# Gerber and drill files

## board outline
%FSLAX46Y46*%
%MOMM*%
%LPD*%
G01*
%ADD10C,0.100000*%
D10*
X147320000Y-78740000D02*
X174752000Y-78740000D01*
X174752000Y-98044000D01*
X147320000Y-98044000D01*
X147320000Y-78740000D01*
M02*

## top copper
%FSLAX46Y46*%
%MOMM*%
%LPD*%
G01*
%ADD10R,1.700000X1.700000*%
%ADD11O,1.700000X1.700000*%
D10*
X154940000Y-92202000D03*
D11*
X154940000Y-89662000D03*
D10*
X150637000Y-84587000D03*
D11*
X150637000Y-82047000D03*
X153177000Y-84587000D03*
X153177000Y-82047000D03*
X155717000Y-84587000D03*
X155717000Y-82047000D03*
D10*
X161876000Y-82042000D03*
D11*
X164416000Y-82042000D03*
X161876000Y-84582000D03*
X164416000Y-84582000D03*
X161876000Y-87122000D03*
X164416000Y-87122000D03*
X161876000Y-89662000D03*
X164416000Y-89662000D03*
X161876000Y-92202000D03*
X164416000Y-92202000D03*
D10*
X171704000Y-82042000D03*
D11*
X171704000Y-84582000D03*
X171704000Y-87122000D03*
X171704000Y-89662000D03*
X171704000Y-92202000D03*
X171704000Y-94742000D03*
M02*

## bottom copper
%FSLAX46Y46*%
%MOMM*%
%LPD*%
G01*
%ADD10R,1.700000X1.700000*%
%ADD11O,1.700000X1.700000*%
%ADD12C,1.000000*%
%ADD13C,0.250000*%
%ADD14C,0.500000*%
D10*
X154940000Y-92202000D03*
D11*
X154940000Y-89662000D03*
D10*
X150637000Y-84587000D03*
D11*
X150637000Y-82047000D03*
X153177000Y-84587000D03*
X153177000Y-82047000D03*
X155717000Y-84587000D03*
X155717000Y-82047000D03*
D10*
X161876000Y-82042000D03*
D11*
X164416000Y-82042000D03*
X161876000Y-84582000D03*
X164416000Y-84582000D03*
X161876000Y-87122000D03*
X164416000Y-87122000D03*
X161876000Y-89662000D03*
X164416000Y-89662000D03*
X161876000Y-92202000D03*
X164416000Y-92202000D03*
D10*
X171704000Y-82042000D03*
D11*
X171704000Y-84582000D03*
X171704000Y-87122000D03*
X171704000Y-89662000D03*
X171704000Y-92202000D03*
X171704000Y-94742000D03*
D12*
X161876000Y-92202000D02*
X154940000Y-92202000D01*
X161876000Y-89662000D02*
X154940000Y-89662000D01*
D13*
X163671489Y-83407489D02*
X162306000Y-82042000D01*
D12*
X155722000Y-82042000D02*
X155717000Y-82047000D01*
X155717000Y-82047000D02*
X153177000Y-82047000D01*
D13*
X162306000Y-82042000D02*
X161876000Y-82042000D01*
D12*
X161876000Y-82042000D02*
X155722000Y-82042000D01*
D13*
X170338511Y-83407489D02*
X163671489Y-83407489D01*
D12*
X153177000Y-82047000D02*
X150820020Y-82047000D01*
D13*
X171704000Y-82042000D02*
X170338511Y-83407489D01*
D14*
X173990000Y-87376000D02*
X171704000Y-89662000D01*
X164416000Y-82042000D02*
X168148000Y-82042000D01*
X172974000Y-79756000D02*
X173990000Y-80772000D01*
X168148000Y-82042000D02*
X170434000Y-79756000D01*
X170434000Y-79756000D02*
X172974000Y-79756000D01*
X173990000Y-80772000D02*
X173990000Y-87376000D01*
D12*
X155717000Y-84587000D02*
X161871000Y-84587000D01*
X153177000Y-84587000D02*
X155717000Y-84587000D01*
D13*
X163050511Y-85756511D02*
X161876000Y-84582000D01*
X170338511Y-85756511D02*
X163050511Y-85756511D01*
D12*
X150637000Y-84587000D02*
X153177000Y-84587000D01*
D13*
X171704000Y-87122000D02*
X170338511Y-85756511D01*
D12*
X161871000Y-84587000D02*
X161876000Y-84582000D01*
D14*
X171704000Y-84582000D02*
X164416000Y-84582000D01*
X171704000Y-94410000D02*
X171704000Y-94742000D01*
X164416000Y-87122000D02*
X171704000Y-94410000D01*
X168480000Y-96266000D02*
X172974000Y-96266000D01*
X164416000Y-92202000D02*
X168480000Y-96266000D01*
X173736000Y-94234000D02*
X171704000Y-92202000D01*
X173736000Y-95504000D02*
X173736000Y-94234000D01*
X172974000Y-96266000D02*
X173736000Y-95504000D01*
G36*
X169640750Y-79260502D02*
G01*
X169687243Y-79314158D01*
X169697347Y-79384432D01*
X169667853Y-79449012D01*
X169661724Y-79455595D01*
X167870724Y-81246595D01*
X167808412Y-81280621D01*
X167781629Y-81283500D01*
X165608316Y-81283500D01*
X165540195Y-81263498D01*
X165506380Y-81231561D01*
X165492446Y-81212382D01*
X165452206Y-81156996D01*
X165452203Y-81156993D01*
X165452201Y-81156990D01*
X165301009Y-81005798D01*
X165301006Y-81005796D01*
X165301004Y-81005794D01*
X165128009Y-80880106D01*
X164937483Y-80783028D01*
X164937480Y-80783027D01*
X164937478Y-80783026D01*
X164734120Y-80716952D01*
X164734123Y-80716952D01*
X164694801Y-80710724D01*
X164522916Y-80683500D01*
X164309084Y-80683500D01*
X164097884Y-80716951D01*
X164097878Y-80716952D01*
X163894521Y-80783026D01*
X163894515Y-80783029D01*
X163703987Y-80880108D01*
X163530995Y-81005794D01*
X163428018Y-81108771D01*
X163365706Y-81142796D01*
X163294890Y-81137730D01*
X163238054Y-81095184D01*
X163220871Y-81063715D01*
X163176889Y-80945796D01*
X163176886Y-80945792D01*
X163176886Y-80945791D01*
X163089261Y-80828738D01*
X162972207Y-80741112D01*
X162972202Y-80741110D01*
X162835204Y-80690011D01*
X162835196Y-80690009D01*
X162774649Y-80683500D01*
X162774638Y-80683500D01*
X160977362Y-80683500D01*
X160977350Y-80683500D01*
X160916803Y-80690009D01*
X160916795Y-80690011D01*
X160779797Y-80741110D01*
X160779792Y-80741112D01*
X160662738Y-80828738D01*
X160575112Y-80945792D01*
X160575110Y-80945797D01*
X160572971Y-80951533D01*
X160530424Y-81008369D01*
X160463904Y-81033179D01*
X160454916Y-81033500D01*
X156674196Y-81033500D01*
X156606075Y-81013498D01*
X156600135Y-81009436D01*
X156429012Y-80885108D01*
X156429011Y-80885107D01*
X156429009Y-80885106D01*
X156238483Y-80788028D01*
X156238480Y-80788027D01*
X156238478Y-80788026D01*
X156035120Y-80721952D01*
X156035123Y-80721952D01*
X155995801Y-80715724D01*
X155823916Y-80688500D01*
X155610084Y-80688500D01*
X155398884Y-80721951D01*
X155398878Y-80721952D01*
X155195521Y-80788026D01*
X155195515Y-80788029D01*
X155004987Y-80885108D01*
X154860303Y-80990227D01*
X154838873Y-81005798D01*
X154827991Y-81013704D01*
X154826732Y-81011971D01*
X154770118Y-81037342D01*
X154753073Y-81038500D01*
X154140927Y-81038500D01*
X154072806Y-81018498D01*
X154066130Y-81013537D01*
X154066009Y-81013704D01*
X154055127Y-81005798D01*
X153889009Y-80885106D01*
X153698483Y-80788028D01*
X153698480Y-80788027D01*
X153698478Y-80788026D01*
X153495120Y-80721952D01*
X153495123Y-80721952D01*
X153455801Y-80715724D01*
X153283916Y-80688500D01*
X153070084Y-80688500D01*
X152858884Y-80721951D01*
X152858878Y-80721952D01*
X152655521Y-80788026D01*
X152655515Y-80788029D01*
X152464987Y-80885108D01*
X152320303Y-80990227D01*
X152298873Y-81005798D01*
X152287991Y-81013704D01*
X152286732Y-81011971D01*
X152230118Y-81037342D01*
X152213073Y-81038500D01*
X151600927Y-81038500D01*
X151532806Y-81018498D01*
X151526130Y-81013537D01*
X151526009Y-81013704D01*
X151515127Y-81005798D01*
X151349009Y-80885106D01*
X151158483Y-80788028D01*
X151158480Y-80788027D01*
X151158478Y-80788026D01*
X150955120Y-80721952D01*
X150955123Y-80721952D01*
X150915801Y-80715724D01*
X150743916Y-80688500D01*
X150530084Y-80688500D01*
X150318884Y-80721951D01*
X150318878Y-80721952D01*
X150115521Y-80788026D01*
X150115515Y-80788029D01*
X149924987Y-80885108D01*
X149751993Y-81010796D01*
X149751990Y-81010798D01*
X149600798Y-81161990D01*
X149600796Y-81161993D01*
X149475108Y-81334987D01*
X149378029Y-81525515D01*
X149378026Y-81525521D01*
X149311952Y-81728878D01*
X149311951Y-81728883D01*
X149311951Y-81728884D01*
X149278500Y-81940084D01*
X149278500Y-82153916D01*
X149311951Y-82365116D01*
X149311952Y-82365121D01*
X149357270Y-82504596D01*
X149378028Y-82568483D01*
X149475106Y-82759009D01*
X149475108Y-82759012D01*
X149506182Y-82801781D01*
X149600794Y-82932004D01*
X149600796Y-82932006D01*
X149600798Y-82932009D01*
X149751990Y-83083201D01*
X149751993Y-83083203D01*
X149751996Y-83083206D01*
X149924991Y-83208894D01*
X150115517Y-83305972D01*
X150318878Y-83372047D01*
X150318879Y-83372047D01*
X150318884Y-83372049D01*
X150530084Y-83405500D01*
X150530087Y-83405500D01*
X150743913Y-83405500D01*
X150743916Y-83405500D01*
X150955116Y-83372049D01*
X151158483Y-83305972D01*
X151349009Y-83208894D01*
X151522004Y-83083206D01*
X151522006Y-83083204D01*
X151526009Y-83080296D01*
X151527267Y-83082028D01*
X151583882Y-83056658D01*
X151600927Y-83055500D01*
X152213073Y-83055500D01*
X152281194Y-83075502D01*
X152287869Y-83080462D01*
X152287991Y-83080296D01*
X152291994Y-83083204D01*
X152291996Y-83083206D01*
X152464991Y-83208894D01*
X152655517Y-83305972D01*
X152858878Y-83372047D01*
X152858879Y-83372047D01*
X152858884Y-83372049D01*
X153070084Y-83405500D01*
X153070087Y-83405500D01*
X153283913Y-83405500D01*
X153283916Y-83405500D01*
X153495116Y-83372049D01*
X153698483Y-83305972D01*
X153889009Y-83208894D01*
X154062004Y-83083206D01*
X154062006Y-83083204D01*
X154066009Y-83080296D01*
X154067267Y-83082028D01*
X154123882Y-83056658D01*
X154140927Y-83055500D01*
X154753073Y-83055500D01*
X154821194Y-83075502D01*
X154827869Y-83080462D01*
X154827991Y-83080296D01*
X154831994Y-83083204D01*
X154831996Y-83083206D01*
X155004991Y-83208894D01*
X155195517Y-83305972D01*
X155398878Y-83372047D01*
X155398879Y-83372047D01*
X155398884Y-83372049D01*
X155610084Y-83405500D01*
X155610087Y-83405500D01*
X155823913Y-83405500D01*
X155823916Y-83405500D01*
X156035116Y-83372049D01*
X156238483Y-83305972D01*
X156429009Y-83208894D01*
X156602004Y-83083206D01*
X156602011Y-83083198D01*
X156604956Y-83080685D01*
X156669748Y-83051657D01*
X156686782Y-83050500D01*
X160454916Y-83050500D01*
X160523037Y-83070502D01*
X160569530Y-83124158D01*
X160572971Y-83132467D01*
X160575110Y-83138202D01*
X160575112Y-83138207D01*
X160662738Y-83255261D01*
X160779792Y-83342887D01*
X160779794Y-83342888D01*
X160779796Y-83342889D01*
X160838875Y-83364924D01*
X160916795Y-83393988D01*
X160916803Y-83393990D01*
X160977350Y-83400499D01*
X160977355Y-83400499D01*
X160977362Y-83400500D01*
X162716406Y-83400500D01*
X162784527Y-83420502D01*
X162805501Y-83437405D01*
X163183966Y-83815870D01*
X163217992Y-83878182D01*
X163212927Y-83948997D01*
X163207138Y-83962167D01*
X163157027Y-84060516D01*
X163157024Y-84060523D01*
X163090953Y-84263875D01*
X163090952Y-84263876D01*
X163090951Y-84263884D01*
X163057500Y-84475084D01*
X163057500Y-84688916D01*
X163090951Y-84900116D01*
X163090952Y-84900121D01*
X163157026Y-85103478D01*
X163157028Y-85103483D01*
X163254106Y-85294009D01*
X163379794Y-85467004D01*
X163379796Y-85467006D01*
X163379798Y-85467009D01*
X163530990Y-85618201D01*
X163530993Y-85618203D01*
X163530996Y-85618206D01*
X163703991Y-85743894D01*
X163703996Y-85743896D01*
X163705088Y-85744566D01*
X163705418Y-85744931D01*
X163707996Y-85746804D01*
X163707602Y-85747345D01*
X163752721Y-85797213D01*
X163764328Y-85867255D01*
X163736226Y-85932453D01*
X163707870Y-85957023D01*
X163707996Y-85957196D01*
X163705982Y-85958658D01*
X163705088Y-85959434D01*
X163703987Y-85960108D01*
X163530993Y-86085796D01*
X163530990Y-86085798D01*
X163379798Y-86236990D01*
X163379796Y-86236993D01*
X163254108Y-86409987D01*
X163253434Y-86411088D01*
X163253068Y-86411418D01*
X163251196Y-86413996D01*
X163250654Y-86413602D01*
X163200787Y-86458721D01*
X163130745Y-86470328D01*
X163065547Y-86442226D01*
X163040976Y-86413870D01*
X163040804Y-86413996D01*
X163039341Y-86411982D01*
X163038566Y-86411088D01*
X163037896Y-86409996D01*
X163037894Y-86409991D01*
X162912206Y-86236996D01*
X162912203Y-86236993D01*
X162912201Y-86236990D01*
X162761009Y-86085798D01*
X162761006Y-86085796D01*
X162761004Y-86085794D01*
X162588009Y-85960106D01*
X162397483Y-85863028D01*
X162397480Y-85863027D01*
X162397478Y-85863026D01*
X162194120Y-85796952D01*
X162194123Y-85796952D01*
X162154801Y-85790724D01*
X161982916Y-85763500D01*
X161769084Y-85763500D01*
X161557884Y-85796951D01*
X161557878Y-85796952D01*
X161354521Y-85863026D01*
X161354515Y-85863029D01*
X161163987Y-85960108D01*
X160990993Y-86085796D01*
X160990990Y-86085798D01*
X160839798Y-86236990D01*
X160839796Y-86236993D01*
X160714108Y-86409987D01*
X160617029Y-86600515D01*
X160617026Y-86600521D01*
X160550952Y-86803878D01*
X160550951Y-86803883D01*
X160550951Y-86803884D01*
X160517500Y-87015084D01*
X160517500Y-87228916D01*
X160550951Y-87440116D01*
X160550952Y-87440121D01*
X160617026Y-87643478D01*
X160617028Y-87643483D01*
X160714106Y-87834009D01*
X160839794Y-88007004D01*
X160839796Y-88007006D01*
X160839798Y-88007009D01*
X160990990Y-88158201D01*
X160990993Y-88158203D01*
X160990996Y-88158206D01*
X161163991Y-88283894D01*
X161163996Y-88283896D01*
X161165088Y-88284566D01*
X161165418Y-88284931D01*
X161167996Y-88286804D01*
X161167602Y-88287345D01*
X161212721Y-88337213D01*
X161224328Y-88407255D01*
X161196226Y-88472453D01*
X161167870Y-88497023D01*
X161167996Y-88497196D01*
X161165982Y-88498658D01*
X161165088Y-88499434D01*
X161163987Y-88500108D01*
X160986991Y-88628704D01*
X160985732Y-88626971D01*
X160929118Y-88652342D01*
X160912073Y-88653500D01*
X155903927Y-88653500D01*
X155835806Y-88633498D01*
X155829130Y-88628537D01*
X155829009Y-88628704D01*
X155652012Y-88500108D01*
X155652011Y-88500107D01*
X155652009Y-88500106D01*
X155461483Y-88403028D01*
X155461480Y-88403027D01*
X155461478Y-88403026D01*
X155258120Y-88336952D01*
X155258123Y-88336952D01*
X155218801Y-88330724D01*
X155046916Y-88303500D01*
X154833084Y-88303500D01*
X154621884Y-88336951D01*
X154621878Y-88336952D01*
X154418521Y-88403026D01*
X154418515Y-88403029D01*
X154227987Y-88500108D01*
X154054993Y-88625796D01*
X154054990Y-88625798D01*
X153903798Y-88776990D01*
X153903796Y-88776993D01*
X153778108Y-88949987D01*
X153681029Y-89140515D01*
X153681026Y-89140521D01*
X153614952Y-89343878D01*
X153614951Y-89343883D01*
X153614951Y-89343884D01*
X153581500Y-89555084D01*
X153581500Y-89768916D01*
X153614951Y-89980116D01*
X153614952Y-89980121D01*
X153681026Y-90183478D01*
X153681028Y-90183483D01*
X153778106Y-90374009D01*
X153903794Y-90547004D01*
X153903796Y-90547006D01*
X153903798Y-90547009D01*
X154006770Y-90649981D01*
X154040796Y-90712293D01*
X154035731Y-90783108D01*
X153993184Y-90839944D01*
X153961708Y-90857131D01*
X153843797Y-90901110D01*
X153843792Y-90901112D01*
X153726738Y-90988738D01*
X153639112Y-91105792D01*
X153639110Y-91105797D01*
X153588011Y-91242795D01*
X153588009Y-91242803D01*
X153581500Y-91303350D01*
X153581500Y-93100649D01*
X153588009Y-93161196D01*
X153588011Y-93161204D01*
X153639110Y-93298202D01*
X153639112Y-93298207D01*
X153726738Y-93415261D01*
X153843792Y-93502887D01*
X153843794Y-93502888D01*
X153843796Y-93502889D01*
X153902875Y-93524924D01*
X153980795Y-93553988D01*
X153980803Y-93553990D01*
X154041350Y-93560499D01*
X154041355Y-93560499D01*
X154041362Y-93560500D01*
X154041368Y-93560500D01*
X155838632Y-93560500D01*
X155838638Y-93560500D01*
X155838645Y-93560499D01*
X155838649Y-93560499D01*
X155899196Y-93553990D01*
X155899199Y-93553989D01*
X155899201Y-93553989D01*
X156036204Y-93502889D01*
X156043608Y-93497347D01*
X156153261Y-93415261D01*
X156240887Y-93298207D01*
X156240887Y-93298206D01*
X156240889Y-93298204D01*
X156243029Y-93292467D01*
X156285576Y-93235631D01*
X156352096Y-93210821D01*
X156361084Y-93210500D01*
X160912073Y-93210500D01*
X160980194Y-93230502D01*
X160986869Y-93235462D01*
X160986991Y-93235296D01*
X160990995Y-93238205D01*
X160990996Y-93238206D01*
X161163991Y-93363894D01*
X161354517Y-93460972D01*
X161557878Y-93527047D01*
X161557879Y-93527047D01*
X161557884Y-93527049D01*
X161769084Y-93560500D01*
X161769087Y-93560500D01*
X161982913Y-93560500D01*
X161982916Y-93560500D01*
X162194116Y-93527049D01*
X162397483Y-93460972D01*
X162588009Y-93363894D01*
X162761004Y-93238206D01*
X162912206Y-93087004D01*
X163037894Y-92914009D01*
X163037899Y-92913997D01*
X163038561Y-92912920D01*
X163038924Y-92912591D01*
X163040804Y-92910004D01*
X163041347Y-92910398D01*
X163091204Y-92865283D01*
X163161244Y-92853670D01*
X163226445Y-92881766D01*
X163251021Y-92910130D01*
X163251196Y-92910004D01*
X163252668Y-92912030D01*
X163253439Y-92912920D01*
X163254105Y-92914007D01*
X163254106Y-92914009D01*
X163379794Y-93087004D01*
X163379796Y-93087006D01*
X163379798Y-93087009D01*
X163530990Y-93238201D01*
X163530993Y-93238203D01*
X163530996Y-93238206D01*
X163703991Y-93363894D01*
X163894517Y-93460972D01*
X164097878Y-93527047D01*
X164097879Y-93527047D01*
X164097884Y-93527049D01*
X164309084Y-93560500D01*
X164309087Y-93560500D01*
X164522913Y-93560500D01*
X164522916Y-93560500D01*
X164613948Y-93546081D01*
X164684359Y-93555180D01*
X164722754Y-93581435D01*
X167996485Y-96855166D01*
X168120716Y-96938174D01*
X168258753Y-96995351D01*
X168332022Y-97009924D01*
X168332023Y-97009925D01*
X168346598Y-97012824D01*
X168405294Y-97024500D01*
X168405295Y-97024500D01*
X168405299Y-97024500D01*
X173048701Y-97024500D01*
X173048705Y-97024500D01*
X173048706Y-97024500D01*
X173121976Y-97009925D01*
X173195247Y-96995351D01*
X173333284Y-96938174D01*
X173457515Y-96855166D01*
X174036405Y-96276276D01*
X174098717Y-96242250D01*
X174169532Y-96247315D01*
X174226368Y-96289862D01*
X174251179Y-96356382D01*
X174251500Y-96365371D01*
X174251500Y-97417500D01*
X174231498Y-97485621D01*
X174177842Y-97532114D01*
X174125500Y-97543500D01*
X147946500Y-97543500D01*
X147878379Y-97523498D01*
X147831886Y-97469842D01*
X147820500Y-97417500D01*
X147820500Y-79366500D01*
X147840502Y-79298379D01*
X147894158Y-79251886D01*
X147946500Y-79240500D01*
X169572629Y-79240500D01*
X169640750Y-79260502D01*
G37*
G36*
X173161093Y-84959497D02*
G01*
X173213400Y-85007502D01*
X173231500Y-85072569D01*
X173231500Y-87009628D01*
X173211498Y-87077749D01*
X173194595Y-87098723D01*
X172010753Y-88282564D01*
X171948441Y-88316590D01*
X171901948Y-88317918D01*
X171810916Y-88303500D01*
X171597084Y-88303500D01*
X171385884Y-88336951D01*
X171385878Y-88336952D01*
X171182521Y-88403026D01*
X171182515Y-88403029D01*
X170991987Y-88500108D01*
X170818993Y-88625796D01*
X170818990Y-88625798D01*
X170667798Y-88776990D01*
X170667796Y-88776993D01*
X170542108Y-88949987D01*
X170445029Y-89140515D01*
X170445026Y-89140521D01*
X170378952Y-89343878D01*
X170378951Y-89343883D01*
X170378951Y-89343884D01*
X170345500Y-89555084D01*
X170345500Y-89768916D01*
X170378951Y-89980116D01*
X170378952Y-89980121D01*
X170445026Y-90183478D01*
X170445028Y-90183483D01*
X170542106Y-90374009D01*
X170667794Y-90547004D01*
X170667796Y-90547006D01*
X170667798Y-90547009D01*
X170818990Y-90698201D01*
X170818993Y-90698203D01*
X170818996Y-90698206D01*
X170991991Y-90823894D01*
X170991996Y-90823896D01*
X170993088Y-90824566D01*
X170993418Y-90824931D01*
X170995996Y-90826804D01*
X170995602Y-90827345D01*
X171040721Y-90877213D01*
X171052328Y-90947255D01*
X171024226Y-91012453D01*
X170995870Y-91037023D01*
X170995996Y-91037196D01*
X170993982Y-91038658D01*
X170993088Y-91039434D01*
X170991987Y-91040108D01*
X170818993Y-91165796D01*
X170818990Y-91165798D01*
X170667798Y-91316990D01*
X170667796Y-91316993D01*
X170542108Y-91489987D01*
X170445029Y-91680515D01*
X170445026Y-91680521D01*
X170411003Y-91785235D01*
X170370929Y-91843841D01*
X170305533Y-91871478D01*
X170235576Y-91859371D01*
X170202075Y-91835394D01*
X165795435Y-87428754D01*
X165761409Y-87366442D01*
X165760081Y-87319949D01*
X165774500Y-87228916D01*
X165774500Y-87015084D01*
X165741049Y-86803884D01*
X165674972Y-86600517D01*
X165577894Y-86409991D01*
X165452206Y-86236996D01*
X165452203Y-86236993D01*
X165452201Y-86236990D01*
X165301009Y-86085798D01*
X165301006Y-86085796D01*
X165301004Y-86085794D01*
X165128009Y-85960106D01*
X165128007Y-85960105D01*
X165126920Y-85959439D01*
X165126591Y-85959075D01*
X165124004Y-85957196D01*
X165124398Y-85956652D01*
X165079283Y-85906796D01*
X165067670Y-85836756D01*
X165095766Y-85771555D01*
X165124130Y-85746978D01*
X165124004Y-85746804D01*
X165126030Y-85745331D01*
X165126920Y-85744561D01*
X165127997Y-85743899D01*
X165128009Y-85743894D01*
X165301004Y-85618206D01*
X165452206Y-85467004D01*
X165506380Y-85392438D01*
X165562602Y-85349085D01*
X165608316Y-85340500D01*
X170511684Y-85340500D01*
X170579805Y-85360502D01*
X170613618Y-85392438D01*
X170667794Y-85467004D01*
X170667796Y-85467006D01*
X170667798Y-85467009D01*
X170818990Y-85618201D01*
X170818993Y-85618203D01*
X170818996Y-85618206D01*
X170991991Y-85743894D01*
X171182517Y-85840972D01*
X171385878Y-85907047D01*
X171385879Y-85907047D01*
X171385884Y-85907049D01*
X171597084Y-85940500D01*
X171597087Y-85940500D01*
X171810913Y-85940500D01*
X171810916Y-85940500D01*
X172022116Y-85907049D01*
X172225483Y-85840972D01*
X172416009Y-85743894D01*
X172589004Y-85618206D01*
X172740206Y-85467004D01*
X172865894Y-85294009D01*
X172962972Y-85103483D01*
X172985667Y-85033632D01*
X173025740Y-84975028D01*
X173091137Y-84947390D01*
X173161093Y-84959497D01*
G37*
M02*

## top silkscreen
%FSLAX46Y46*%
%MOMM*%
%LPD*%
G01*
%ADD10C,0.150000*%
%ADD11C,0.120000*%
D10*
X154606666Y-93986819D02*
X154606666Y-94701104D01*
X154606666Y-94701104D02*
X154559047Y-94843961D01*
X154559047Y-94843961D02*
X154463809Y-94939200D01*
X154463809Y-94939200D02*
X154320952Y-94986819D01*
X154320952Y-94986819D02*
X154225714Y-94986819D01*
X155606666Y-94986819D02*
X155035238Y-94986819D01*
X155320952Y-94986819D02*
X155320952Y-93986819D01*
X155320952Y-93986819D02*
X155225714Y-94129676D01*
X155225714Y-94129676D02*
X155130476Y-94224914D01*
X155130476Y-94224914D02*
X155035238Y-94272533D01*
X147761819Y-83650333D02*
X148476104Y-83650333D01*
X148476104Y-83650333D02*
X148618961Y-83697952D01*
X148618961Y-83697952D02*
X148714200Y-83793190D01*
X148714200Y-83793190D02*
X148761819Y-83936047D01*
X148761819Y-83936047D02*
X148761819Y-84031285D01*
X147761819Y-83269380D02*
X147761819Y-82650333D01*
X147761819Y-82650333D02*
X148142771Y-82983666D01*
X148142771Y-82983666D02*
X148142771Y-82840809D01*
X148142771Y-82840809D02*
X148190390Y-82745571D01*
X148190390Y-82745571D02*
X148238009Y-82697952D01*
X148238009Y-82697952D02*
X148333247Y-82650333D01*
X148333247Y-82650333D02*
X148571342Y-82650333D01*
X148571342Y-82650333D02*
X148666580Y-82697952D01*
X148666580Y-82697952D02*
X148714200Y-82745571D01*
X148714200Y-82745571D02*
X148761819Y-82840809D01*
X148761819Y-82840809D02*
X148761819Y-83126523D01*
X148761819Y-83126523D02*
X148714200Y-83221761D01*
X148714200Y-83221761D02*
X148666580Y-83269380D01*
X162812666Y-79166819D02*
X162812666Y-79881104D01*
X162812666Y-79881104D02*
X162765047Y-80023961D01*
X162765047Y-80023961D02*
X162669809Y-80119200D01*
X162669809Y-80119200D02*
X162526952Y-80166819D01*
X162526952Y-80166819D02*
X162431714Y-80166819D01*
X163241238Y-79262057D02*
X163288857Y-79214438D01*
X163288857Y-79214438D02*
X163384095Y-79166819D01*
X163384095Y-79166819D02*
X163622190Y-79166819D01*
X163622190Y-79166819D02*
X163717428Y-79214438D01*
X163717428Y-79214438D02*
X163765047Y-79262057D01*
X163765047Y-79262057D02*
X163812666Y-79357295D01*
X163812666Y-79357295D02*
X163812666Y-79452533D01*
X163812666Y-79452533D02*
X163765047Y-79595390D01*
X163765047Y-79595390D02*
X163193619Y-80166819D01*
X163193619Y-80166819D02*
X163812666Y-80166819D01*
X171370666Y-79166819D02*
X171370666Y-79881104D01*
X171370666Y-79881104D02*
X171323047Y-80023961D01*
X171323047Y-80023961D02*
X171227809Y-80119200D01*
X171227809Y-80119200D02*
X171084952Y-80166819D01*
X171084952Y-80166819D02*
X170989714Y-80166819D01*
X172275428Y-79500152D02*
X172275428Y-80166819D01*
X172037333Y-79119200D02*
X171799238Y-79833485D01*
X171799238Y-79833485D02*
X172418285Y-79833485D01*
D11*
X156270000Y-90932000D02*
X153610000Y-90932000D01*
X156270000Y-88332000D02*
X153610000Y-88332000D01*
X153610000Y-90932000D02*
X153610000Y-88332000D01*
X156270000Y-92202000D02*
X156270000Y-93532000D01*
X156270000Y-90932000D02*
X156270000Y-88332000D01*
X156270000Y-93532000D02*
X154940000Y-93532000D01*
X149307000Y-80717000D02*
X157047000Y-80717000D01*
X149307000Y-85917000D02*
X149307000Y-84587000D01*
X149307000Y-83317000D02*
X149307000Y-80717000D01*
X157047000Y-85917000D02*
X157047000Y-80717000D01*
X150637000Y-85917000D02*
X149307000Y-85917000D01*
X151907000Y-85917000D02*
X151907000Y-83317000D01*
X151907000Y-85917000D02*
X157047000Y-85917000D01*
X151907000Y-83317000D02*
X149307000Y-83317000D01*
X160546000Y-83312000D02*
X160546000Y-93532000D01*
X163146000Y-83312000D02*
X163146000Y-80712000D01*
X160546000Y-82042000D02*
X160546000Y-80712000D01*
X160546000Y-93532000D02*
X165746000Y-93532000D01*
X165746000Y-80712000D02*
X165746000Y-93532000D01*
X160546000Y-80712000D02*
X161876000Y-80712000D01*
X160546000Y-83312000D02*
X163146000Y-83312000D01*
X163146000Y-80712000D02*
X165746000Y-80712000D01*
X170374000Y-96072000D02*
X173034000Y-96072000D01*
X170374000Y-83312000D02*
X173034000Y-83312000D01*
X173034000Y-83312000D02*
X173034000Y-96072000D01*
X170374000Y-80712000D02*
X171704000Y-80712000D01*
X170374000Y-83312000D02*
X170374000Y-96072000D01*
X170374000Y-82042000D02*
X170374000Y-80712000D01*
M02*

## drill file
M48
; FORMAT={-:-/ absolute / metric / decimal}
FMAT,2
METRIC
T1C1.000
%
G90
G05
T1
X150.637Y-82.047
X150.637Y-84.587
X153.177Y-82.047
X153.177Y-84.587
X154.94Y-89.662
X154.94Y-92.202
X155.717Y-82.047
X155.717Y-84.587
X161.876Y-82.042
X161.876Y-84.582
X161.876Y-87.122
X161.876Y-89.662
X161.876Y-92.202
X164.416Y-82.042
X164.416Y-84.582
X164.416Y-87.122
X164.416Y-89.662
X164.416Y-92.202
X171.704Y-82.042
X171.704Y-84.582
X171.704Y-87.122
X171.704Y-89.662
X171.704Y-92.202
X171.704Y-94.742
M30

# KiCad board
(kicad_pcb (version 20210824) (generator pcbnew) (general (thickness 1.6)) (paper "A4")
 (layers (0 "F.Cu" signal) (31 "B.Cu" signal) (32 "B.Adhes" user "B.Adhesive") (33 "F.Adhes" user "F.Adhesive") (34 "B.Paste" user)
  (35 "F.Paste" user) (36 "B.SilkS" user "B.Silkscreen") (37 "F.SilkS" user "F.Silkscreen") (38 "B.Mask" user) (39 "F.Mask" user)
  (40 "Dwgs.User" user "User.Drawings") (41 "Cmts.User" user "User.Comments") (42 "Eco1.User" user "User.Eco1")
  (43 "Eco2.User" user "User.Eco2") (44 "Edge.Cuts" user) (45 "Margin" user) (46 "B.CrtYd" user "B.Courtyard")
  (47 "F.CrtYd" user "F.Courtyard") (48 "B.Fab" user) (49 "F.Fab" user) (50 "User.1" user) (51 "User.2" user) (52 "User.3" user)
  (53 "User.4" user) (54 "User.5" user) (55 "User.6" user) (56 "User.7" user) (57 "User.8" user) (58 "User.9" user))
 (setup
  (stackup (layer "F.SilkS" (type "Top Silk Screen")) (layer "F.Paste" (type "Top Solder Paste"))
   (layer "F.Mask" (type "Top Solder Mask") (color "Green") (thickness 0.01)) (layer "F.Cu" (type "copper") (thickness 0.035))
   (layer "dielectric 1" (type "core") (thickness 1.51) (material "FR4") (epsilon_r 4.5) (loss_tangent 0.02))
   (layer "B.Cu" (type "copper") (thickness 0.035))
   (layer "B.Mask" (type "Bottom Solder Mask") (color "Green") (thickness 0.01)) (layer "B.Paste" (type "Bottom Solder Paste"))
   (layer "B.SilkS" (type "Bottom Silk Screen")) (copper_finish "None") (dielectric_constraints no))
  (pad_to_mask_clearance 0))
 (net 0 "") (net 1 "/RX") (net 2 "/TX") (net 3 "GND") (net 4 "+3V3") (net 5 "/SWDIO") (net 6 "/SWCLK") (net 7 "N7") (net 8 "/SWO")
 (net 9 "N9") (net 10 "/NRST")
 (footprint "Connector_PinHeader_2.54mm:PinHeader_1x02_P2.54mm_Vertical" (layer "F.Cu") (at 154.94 92.202 180)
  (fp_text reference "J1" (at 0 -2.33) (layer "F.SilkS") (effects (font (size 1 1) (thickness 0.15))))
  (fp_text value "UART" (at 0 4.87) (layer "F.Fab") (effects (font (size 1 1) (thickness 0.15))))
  (fp_line (start -1.33 1.27) (end 1.33 1.27) (layer "F.SilkS") (width 0.12))
  (fp_line (start -1.33 3.87) (end 1.33 3.87) (layer "F.SilkS") (width 0.12))
  (fp_line (start 1.33 1.27) (end 1.33 3.87) (layer "F.SilkS") (width 0.12))
  (fp_line (start -1.33 0) (end -1.33 -1.33) (layer "F.SilkS") (width 0.12))
  (fp_line (start -1.33 1.27) (end -1.33 3.87) (layer "F.SilkS") (width 0.12))
  (fp_line (start -1.33 -1.33) (end 0 -1.33) (layer "F.SilkS") (width 0.12))
  (pad "1" thru_hole rect locked (at 0 0 180) (size 1.7 1.7) (drill 1) (layers *.Cu *.Mask) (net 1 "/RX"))
  (pad "2" thru_hole oval locked (at 0 2.54 180) (size 1.7 1.7) (drill 1) (layers *.Cu *.Mask) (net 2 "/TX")))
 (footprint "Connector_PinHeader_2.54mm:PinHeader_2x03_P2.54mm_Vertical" (layer "F.Cu") (at 150.637 84.587 90)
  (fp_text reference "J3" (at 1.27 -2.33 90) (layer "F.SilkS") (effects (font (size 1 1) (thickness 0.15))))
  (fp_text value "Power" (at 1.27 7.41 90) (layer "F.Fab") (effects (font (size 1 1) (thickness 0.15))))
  (fp_line (start 3.87 -1.33) (end 3.87 6.41) (layer "F.SilkS") (width 0.12))
  (fp_line (start -1.33 -1.33) (end 0 -1.33) (layer "F.SilkS") (width 0.12))
  (fp_line (start 1.27 -1.33) (end 3.87 -1.33) (layer "F.SilkS") (width 0.12))
  (fp_line (start -1.33 6.41) (end 3.87 6.41) (layer "F.SilkS") (width 0.12))
  (fp_line (start -1.33 0) (end -1.33 -1.33) (layer "F.SilkS") (width 0.12))
  (fp_line (start -1.33 1.27) (end 1.27 1.27) (layer "F.SilkS") (width 0.12))
  (fp_line (start -1.33 1.27) (end -1.33 6.41) (layer "F.SilkS") (width 0.12))
  (fp_line (start 1.27 1.27) (end 1.27 -1.33) (layer "F.SilkS") (width 0.12))
  (pad "1" thru_hole rect locked (at 0 0 90) (size 1.7 1.7) (drill 1) (layers *.Cu *.Mask) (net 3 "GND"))
  (pad "2" thru_hole oval locked (at 2.54 0 90) (size 1.7 1.7) (drill 1) (layers *.Cu *.Mask) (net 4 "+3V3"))
  (pad "3" thru_hole oval locked (at 0 2.54 90) (size 1.7 1.7) (drill 1) (layers *.Cu *.Mask) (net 3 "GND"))
  (pad "4" thru_hole oval locked (at 2.54 2.54 90) (size 1.7 1.7) (drill 1) (layers *.Cu *.Mask) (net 4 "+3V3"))
  (pad "5" thru_hole oval locked (at 0 5.08 90) (size 1.7 1.7) (drill 1) (layers *.Cu *.Mask) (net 3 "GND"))
  (pad "6" thru_hole oval locked (at 2.54 5.08 90) (size 1.7 1.7) (drill 1) (layers *.Cu *.Mask) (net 4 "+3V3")))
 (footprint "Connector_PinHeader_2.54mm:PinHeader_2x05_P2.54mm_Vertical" (layer "F.Cu") (at 161.876 82.042)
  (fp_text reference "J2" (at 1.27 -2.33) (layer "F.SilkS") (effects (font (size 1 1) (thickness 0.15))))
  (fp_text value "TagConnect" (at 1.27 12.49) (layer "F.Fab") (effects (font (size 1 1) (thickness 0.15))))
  (fp_line (start -1.33 1.27) (end -1.33 11.49) (layer "F.SilkS") (width 0.12))
  (fp_line (start 1.27 1.27) (end 1.27 -1.33) (layer "F.SilkS") (width 0.12))
  (fp_line (start -1.33 0) (end -1.33 -1.33) (layer "F.SilkS") (width 0.12))
  (fp_line (start -1.33 11.49) (end 3.87 11.49) (layer "F.SilkS") (width 0.12))
  (fp_line (start 3.87 -1.33) (end 3.87 11.49) (layer "F.SilkS") (width 0.12))
  (fp_line (start -1.33 -1.33) (end 0 -1.33) (layer "F.SilkS") (width 0.12))
  (fp_line (start -1.33 1.27) (end 1.27 1.27) (layer "F.SilkS") (width 0.12))
  (fp_line (start 1.27 -1.33) (end 3.87 -1.33) (layer "F.SilkS") (width 0.12))
  (pad "1" thru_hole rect locked (at 0 0) (size 1.7 1.7) (drill 1) (layers *.Cu *.Mask) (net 4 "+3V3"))
  (pad "2" thru_hole oval locked (at 2.54 0) (size 1.7 1.7) (drill 1) (layers *.Cu *.Mask) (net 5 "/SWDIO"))
  (pad "3" thru_hole oval locked (at 0 2.54) (size 1.7 1.7) (drill 1) (layers *.Cu *.Mask) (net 3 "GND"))
  (pad "4" thru_hole oval locked (at 2.54 2.54) (size 1.7 1.7) (drill 1) (layers *.Cu *.Mask) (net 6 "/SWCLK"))
  (pad "5" thru_hole oval locked (at 0 5.08) (size 1.7 1.7) (drill 1) (layers *.Cu *.Mask) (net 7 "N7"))
  (pad "6" thru_hole oval locked (at 2.54 5.08) (size 1.7 1.7) (drill 1) (layers *.Cu *.Mask) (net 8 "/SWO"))
  (pad "7" thru_hole oval locked (at 0 7.62) (size 1.7 1.7) (drill 1) (layers *.Cu *.Mask) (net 2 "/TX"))
  (pad "8" thru_hole oval locked (at 2.54 7.62) (size 1.7 1.7) (drill 1) (layers *.Cu *.Mask) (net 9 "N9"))
  (pad "9" thru_hole oval locked (at 0 10.16) (size 1.7 1.7) (drill 1) (layers *.Cu *.Mask) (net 1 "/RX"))
  (pad "10" thru_hole oval locked (at 2.54 10.16) (size 1.7 1.7) (drill 1) (layers *.Cu *.Mask) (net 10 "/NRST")))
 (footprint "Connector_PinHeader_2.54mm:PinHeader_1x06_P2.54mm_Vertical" (layer "F.Cu") (at 171.704 82.042)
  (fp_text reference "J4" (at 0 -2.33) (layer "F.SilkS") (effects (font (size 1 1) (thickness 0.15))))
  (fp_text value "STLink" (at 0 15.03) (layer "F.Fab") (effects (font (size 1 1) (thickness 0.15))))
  (fp_line (start -1.33 14.03) (end 1.33 14.03) (layer "F.SilkS") (width 0.12))
  (fp_line (start -1.33 1.27) (end 1.33 1.27) (layer "F.SilkS") (width 0.12))
  (fp_line (start 1.33 1.27) (end 1.33 14.03) (layer "F.SilkS") (width 0.12))
  (fp_line (start -1.33 -1.33) (end 0 -1.33) (layer "F.SilkS") (width 0.12))
  (fp_line (start -1.33 1.27) (end -1.33 14.03) (layer "F.SilkS") (width 0.12))
  (fp_line (start -1.33 0) (end -1.33 -1.33) (layer "F.SilkS") (width 0.12))
  (pad "1" thru_hole rect locked (at 0 0) (size 1.7 1.7) (drill 1) (layers *.Cu *.Mask) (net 4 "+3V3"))
  (pad "2" thru_hole oval locked (at 0 2.54) (size 1.7 1.7) (drill 1) (layers *.Cu *.Mask) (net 6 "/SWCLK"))
  (pad "3" thru_hole oval locked (at 0 5.08) (size 1.7 1.7) (drill 1) (layers *.Cu *.Mask) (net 3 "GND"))
  (pad "4" thru_hole oval locked (at 0 7.62) (size 1.7 1.7) (drill 1) (layers *.Cu *.Mask) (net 5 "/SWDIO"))
  (pad "5" thru_hole oval locked (at 0 10.16) (size 1.7 1.7) (drill 1) (layers *.Cu *.Mask) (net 10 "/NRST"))
  (pad "6" thru_hole oval locked (at 0 12.7) (size 1.7 1.7) (drill 1) (layers *.Cu *.Mask) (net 8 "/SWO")))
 (gr_rect (start 147.32 78.74) (end 174.752 98.044) (layer "Edge.Cuts") (width 0.1) (fill none))
 (segment (start 161.876 92.202) (end 154.94 92.202) (width 1) (layer "B.Cu") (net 1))
 (segment (start 161.876 89.662) (end 154.94 89.662) (width 1) (layer "B.Cu") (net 2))
 (segment (start 163.671489 83.407489) (end 162.306 82.042) (width 0.25) (layer "B.Cu") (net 4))
 (segment (start 155.722 82.042) (end 155.717 82.047) (width 1) (layer "B.Cu") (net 4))
 (segment (start 155.717 82.047) (end 153.177 82.047) (width 1) (layer "B.Cu") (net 4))
 (segment (start 162.306 82.042) (end 161.876 82.042) (width 0.25) (layer "B.Cu") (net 4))
 (segment (start 161.876 82.042) (end 155.722 82.042) (width 1) (layer "B.Cu") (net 4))
 (segment (start 170.338511 83.407489) (end 163.671489 83.407489) (width 0.25) (layer "B.Cu") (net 4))
 (segment (start 153.177 82.047) (end 150.82002 82.047) (width 1) (layer "B.Cu") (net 4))
 (segment (start 171.704 82.042) (end 170.338511 83.407489) (width 0.25) (layer "B.Cu") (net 4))
 (segment (start 173.99 87.376) (end 171.704 89.662) (width 0.5) (layer "B.Cu") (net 5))
 (segment (start 164.416 82.042) (end 168.148 82.042) (width 0.5) (layer "B.Cu") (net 5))
 (segment (start 172.974 79.756) (end 173.99 80.772) (width 0.5) (layer "B.Cu") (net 5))
 (segment (start 168.148 82.042) (end 170.434 79.756) (width 0.5) (layer "B.Cu") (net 5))
 (segment (start 170.434 79.756) (end 172.974 79.756) (width 0.5) (layer "B.Cu") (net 5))
 (segment (start 173.99 80.772) (end 173.99 87.376) (width 0.5) (layer "B.Cu") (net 5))
 (segment (start 155.717 84.587) (end 161.871 84.587) (width 1) (layer "B.Cu") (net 3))
 (segment (start 153.177 84.587) (end 155.717 84.587) (width 1) (layer "B.Cu") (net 3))
 (segment (start 163.050511 85.756511) (end 161.876 84.582) (width 0.25) (layer "B.Cu") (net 3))
 (segment (start 170.338511 85.756511) (end 163.050511 85.756511) (width 0.25) (layer "B.Cu") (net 3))
 (segment (start 150.637 84.587) (end 153.177 84.587) (width 1) (layer "B.Cu") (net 3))
 (segment (start 171.704 87.122) (end 170.338511 85.756511) (width 0.25) (layer "B.Cu") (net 3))
 (segment (start 161.871 84.587) (end 161.876 84.582) (width 1) (layer "B.Cu") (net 3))
 (segment (start 171.704 84.582) (end 164.416 84.582) (width 0.5) (layer "B.Cu") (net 6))
 (segment (start 171.704 94.41) (end 171.704 94.742) (width 0.5) (layer "B.Cu") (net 8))
 (segment (start 164.416 87.122) (end 171.704 94.41) (width 0.5) (layer "B.Cu") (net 8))
 (segment (start 168.48 96.266) (end 172.974 96.266) (width 0.5) (layer "B.Cu") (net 10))
 (segment (start 164.416 92.202) (end 168.48 96.266) (width 0.5) (layer "B.Cu") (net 10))
 (segment (start 173.736 94.234) (end 171.704 92.202) (width 0.5) (layer "B.Cu") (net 10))
 (segment (start 173.736 95.504) (end 173.736 94.234) (width 0.5) (layer "B.Cu") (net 10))
 (segment (start 172.974 96.266) (end 173.736 95.504) (width 0.5) (layer "B.Cu") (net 10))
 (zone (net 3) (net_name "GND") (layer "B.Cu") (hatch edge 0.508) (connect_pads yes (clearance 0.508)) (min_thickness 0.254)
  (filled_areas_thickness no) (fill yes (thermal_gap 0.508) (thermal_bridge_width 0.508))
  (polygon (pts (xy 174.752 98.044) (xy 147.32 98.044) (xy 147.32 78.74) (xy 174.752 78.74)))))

